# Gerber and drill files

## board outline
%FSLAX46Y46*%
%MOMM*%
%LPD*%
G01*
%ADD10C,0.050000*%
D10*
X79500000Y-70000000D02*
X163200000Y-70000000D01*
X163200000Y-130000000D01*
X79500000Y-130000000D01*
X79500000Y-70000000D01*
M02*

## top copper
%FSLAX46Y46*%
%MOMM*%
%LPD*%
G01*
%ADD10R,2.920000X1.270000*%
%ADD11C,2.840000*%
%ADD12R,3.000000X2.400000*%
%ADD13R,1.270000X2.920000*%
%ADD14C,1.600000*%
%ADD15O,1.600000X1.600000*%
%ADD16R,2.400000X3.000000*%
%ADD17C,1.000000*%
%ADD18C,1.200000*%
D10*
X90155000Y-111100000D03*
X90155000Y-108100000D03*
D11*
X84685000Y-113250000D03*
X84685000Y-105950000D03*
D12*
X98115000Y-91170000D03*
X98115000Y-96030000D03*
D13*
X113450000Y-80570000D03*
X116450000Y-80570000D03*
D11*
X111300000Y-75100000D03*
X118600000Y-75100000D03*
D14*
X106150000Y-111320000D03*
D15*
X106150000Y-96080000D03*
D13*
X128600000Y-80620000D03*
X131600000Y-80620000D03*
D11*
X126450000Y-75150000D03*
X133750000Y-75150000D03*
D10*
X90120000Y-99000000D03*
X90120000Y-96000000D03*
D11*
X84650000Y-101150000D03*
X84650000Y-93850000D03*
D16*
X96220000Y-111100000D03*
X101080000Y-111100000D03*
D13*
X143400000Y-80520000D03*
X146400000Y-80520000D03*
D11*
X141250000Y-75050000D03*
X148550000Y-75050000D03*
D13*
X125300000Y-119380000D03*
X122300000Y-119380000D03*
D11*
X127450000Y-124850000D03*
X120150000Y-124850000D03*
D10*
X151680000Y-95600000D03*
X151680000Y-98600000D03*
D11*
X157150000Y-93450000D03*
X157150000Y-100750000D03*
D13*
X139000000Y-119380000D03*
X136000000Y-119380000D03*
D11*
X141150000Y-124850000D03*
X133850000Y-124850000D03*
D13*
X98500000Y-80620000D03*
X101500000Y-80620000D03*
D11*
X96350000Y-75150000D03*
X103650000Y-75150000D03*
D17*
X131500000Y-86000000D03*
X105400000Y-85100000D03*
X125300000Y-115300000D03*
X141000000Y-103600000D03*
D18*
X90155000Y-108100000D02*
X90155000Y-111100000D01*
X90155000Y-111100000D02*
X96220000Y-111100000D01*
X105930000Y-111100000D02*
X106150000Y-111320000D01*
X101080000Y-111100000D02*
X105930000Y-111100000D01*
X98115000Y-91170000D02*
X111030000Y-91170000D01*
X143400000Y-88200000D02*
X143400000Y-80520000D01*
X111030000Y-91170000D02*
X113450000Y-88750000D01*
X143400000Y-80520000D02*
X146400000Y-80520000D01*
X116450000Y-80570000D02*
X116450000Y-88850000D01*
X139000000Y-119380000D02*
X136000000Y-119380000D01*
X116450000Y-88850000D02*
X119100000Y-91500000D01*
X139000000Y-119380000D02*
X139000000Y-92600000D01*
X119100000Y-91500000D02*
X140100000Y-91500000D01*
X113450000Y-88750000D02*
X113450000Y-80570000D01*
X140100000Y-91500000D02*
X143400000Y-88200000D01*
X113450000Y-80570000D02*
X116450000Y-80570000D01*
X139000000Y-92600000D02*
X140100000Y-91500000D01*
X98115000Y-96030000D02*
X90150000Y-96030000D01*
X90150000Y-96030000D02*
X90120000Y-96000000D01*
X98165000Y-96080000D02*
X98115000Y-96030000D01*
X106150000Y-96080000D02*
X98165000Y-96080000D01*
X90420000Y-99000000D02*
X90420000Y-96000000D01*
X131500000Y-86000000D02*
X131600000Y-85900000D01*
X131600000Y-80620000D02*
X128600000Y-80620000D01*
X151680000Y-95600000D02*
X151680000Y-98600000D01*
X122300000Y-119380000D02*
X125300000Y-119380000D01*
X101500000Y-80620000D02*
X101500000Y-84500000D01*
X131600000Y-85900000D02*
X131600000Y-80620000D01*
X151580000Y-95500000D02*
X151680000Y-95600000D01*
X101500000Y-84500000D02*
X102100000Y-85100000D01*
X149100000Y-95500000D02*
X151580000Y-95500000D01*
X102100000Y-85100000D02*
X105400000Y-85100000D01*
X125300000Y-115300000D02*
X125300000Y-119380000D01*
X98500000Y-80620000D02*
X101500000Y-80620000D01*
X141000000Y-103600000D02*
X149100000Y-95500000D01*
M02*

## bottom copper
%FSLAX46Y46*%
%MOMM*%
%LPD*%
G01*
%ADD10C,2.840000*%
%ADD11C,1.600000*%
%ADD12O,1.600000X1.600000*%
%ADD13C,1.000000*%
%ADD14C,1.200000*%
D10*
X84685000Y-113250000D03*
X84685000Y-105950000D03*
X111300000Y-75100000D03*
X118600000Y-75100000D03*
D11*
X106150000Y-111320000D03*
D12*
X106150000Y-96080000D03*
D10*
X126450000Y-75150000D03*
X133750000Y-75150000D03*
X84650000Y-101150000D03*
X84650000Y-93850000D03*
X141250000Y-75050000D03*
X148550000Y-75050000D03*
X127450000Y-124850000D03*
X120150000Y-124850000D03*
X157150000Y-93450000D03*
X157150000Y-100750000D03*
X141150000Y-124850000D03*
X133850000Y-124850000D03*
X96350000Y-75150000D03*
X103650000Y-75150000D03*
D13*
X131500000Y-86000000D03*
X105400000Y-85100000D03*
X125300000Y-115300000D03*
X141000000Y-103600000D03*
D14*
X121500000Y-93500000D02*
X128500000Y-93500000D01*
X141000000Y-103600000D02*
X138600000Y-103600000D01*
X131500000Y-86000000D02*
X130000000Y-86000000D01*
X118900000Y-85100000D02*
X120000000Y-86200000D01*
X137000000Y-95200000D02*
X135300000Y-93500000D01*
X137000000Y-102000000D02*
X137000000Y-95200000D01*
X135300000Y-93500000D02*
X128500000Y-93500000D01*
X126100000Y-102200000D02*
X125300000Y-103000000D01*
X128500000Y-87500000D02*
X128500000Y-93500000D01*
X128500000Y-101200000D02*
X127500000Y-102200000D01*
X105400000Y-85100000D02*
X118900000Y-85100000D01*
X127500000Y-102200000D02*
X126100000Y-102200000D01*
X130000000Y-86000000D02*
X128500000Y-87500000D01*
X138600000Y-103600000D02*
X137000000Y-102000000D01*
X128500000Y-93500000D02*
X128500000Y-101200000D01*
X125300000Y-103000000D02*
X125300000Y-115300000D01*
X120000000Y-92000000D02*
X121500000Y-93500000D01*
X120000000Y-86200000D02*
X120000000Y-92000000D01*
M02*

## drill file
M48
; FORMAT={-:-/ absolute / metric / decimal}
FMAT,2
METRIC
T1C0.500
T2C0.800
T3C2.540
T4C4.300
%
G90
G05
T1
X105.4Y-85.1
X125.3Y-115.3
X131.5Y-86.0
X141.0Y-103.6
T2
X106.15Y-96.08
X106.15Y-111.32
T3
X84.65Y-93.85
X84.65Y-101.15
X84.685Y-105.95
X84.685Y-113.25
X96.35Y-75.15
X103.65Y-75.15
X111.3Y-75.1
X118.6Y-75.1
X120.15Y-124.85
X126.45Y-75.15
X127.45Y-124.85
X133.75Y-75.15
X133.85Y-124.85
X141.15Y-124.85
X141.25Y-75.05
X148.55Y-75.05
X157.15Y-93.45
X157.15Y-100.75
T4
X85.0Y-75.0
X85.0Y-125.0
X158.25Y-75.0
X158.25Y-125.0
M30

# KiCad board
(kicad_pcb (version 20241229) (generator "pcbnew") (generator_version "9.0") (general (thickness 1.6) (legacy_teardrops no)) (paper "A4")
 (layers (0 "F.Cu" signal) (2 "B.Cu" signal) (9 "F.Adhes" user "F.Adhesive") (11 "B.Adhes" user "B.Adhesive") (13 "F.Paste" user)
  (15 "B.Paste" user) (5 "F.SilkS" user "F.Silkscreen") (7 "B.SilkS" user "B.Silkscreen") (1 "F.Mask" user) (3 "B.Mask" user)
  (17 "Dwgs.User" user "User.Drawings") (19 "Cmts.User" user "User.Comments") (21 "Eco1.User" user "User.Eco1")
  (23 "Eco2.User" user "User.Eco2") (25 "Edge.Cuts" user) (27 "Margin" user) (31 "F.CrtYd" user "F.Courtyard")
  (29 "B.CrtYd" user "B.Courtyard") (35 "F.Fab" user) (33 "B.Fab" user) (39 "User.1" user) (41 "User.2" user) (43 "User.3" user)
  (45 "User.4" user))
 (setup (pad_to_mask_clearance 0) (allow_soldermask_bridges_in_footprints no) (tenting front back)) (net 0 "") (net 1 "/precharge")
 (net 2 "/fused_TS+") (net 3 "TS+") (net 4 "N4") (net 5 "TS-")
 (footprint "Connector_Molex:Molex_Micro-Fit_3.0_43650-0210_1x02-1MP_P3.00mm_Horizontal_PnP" (layer "F.Cu") (at 85.035 109.6 90)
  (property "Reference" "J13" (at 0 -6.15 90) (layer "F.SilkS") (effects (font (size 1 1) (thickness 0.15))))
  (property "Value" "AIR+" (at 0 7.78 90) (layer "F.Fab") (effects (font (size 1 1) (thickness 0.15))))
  (pad "1" smd rect (at -1.5 5.12 90) (size 1.27 2.92) (layers "F.Cu" "F.Mask" "F.Paste") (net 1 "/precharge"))
  (pad "2" smd rect (at 1.5 5.12 90) (size 1.27 2.92) (layers "F.Cu" "F.Mask" "F.Paste") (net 1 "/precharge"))
  (pad "MP" thru_hole circle (at -3.65 -0.35 90) (size 2.84 2.84) (drill 2.54) (layers "*.Cu" "*.Mask") (remove_unused_layers no))
  (pad "MP" thru_hole circle (at 3.65 -0.35 90) (size 2.84 2.84) (drill 2.54) (layers "*.Cu" "*.Mask") (remove_unused_layers no)))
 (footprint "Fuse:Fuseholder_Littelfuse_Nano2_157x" (layer "F.Cu") (at 98.115 93.6 -90)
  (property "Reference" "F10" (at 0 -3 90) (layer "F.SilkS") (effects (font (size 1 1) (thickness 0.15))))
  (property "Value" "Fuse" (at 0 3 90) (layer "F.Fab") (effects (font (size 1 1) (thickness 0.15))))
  (pad "1" smd rect (at -2.43 0 270) (size 2.4 3) (layers "F.Cu" "F.Mask" "F.Paste") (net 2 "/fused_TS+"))
  (pad "2" smd rect (at 2.43 0 270) (size 2.4 3) (layers "F.Cu" "F.Mask" "F.Paste") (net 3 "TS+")))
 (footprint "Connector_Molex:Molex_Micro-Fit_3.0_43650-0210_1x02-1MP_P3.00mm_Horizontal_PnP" (layer "F.Cu") (at 114.95 75.45)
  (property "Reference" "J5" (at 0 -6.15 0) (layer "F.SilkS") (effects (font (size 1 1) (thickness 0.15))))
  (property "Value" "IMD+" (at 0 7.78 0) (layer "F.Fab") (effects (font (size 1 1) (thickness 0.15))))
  (pad "1" smd rect (at -1.5 5.12) (size 1.27 2.92) (layers "F.Cu" "F.Mask" "F.Paste") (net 2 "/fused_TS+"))
  (pad "2" smd rect (at 1.5 5.12) (size 1.27 2.92) (layers "F.Cu" "F.Mask" "F.Paste") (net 2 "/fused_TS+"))
  (pad "MP" thru_hole circle (at -3.65 -0.35) (size 2.84 2.84) (drill 2.54) (layers "*.Cu" "*.Mask") (remove_unused_layers no))
  (pad "MP" thru_hole circle (at 3.65 -0.35) (size 2.84 2.84) (drill 2.54) (layers "*.Cu" "*.Mask") (remove_unused_layers no)))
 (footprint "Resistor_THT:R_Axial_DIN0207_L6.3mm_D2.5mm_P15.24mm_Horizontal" (layer "F.Cu") (at 106.15 111.32 90)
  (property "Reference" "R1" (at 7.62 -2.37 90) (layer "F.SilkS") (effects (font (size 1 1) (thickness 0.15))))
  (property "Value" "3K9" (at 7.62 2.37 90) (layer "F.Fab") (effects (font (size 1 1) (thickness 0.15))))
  (pad "1" thru_hole circle (at 0 0 90) (size 1.6 1.6) (drill 0.8) (layers "*.Cu" "*.Mask") (remove_unused_layers no) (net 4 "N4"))
  (pad "2" thru_hole oval (at 15.24 0 90) (size 1.6 1.6) (drill 0.8) (layers "*.Cu" "*.Mask") (remove_unused_layers no) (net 3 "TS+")))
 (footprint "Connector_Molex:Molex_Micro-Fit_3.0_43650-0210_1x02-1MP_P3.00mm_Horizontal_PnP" (layer "F.Cu") (at 130.1 75.5)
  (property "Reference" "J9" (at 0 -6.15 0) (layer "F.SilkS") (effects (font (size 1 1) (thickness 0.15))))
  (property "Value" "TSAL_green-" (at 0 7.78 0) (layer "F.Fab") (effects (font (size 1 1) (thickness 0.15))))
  (pad "1" smd rect (at -1.5 5.12) (size 1.27 2.92) (layers "F.Cu" "F.Mask" "F.Paste") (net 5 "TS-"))
  (pad "2" smd rect (at 1.5 5.12) (size 1.27 2.92) (layers "F.Cu" "F.Mask" "F.Paste") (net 5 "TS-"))
  (pad "MP" thru_hole circle (at -3.65 -0.35) (size 2.84 2.84) (drill 2.54) (layers "*.Cu" "*.Mask") (remove_unused_layers no))
  (pad "MP" thru_hole circle (at 3.65 -0.35) (size 2.84 2.84) (drill 2.54) (layers "*.Cu" "*.Mask") (remove_unused_layers no)))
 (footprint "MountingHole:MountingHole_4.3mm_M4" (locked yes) (layer "F.Cu") (at 85 75)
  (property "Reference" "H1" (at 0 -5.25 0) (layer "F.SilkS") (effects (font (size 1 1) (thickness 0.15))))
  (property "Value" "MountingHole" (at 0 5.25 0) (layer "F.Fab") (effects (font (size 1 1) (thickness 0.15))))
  (pad "" np_thru_hole circle (at 0 0) (size 4.3 4.3) (drill 4.3) (layers "*.Cu" "*.Mask")))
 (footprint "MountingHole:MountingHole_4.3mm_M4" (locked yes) (layer "F.Cu") (at 85 125)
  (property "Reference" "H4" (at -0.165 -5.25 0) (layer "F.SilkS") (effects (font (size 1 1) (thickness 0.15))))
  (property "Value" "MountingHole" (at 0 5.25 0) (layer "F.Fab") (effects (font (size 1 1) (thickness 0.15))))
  (pad "" np_thru_hole circle (at 0 0) (size 4.3 4.3) (drill 4.3) (layers "*.Cu" "*.Mask")))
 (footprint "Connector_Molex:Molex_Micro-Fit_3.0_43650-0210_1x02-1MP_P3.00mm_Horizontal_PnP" (layer "F.Cu") (at 85 97.5 90)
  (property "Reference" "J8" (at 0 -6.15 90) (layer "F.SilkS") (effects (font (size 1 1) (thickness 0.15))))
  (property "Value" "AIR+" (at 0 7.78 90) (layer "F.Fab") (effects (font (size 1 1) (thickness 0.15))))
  (pad "1" smd rect (at -1.5 5.12 90) (size 1.27 2.92) (layers "F.Cu" "F.Mask" "F.Paste") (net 3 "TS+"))
  (pad "2" smd rect (at 1.5 5.12 90) (size 1.27 2.92) (layers "F.Cu" "F.Mask" "F.Paste") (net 3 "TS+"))
  (pad "MP" thru_hole circle (at -3.65 -0.35 90) (size 2.84 2.84) (drill 2.54) (layers "*.Cu" "*.Mask") (remove_unused_layers no))
  (pad "MP" thru_hole circle (at 3.65 -0.35 90) (size 2.84 2.84) (drill 2.54) (layers "*.Cu" "*.Mask") (remove_unused_layers no)))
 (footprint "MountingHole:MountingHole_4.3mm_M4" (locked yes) (layer "F.Cu") (at 158.25 75)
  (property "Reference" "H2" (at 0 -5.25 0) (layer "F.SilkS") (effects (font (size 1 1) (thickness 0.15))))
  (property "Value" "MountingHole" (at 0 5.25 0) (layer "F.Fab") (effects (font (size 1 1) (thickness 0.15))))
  (pad "" np_thru_hole circle (at 0 0) (size 4.3 4.3) (drill 4.3) (layers "*.Cu" "*.Mask")))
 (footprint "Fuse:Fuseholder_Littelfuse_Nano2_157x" (layer "F.Cu") (at 98.65 111.1)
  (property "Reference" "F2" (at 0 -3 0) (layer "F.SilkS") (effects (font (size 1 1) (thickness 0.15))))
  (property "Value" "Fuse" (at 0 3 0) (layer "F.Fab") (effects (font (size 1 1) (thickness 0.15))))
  (pad "1" smd rect (at -2.43 0) (size 2.4 3) (layers "F.Cu" "F.Mask" "F.Paste") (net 1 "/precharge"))
  (pad "2" smd rect (at 2.43 0) (size 2.4 3) (layers "F.Cu" "F.Mask" "F.Paste") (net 4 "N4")))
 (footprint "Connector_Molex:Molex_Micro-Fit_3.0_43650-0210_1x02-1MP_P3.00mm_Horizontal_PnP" (layer "F.Cu") (at 144.9 75.4)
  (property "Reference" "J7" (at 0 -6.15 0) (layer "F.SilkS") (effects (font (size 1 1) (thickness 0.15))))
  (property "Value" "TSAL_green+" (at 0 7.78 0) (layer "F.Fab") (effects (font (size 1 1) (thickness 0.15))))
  (pad "1" smd rect (at -1.5 5.12) (size 1.27 2.92) (layers "F.Cu" "F.Mask" "F.Paste") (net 2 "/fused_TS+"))
  (pad "2" smd rect (at 1.5 5.12) (size 1.27 2.92) (layers "F.Cu" "F.Mask" "F.Paste") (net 2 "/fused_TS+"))
  (pad "MP" thru_hole circle (at -3.65 -0.35) (size 2.84 2.84) (drill 2.54) (layers "*.Cu" "*.Mask") (remove_unused_layers no))
  (pad "MP" thru_hole circle (at 3.65 -0.35) (size 2.84 2.84) (drill 2.54) (layers "*.Cu" "*.Mask") (remove_unused_layers no)))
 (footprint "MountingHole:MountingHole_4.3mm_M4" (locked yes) (layer "F.Cu") (at 158.25 125)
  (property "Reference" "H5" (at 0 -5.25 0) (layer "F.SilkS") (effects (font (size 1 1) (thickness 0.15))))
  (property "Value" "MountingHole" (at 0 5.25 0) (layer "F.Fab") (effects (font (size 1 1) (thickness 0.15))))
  (pad "" np_thru_hole circle (at 0 0) (size 4.3 4.3) (drill 4.3) (layers "*.Cu" "*.Mask")))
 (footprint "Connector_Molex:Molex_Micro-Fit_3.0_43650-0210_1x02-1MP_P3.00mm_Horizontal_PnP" (layer "F.Cu") (at 123.8 124.5 180)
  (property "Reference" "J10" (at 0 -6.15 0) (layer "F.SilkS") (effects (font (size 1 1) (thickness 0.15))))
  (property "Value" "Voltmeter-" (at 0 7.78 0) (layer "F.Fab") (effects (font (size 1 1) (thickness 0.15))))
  (pad "1" smd rect (at -1.5 5.12 180) (size 1.27 2.92) (layers "F.Cu" "F.Mask" "F.Paste") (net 5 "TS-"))
  (pad "2" smd rect (at 1.5 5.12 180) (size 1.27 2.92) (layers "F.Cu" "F.Mask" "F.Paste") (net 5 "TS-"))
  (pad "MP" thru_hole circle (at -3.65 -0.35 180) (size 2.84 2.84) (drill 2.54) (layers "*.Cu" "*.Mask") (remove_unused_layers no))
  (pad "MP" thru_hole circle (at 3.65 -0.35 180) (size 2.84 2.84) (drill 2.54) (layers "*.Cu" "*.Mask") (remove_unused_layers no)))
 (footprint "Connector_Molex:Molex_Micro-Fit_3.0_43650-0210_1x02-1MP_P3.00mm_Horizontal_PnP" (layer "F.Cu") (at 156.8 97.1 -90)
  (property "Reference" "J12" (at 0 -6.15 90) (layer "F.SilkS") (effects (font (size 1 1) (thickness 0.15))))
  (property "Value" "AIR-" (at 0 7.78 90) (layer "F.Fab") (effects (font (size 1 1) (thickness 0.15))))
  (pad "1" smd rect (at -1.5 5.12 270) (size 1.27 2.92) (layers "F.Cu" "F.Mask" "F.Paste") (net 5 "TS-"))
  (pad "2" smd rect (at 1.5 5.12 270) (size 1.27 2.92) (layers "F.Cu" "F.Mask" "F.Paste") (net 5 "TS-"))
  (pad "MP" thru_hole circle (at -3.65 -0.35 270) (size 2.84 2.84) (drill 2.54) (layers "*.Cu" "*.Mask") (remove_unused_layers no))
  (pad "MP" thru_hole circle (at 3.65 -0.35 270) (size 2.84 2.84) (drill 2.54) (layers "*.Cu" "*.Mask") (remove_unused_layers no)))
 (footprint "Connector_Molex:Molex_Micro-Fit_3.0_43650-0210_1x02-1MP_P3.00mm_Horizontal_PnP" (layer "F.Cu") (at 137.5 124.5 180)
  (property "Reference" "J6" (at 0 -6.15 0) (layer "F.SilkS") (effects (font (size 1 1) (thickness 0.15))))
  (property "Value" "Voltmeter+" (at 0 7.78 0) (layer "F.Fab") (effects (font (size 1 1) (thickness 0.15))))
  (pad "1" smd rect (at -1.5 5.12 180) (size 1.27 2.92) (layers "F.Cu" "F.Mask" "F.Paste") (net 2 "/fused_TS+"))
  (pad "2" smd rect (at 1.5 5.12 180) (size 1.27 2.92) (layers "F.Cu" "F.Mask" "F.Paste") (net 2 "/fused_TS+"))
  (pad "MP" thru_hole circle (at -3.65 -0.35 180) (size 2.84 2.84) (drill 2.54) (layers "*.Cu" "*.Mask") (remove_unused_layers no))
  (pad "MP" thru_hole circle (at 3.65 -0.35 180) (size 2.84 2.84) (drill 2.54) (layers "*.Cu" "*.Mask") (remove_unused_layers no)))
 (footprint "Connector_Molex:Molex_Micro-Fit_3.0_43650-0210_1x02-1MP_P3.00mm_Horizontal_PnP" (layer "F.Cu") (at 100 75.5)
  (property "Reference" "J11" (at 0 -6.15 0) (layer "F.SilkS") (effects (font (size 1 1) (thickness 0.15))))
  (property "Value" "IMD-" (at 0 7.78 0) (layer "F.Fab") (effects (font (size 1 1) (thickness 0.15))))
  (pad "1" smd rect (at -1.5 5.12) (size 1.27 2.92) (layers "F.Cu" "F.Mask" "F.Paste") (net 5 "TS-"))
  (pad "2" smd rect (at 1.5 5.12) (size 1.27 2.92) (layers "F.Cu" "F.Mask" "F.Paste") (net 5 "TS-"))
  (pad "MP" thru_hole circle (at -3.65 -0.35) (size 2.84 2.84) (drill 2.54) (layers "*.Cu" "*.Mask") (remove_unused_layers no))
  (pad "MP" thru_hole circle (at 3.65 -0.35) (size 2.84 2.84) (drill 2.54) (layers "*.Cu" "*.Mask") (remove_unused_layers no)))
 (gr_rect (start 79.5 70) (end 163.2 130) (stroke (width 0.05) (type default)) (fill no) (layer "Edge.Cuts"))
 (segment (start 90.155 108.1) (end 90.155 111.1) (width 1.2) (layer "F.Cu") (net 1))
 (segment (start 90.155 111.1) (end 96.22 111.1) (width 1.2) (layer "F.Cu") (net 1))
 (segment (start 105.93 111.1) (end 106.15 111.32) (width 1.2) (layer "F.Cu") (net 4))
 (segment (start 101.08 111.1) (end 105.93 111.1) (width 1.2) (layer "F.Cu") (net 4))
 (segment (start 98.115 91.17) (end 111.03 91.17) (width 1.2) (layer "F.Cu") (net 2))
 (segment (start 143.4 88.2) (end 143.4 80.52) (width 1.2) (layer "F.Cu") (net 2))
 (segment (start 111.03 91.17) (end 113.45 88.75) (width 1.2) (layer "F.Cu") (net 2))
 (segment (start 143.4 80.52) (end 146.4 80.52) (width 1.2) (layer "F.Cu") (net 2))
 (segment (start 116.45 80.57) (end 116.45 88.85) (width 1.2) (layer "F.Cu") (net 2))
 (segment (start 139 119.38) (end 136 119.38) (width 1.2) (layer "F.Cu") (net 2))
 (segment (start 116.45 88.85) (end 119.1 91.5) (width 1.2) (layer "F.Cu") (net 2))
 (segment (start 139 119.38) (end 139 92.6) (width 1.2) (layer "F.Cu") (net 2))
 (segment (start 119.1 91.5) (end 140.1 91.5) (width 1.2) (layer "F.Cu") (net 2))
 (segment (start 113.45 88.75) (end 113.45 80.57) (width 1.2) (layer "F.Cu") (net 2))
 (segment (start 140.1 91.5) (end 143.4 88.2) (width 1.2) (layer "F.Cu") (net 2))
 (segment (start 113.45 80.57) (end 116.45 80.57) (width 1.2) (layer "F.Cu") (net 2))
 (segment (start 139 92.6) (end 140.1 91.5) (width 1.2) (layer "F.Cu") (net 2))
 (segment (start 98.115 96.03) (end 90.15 96.03) (width 1.2) (layer "F.Cu") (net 3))
 (segment (start 90.15 96.03) (end 90.12 96) (width 1.2) (layer "F.Cu") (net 3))
 (segment (start 98.165 96.08) (end 98.115 96.03) (width 1.2) (layer "F.Cu") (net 3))
 (segment (start 106.15 96.08) (end 98.165 96.08) (width 1.2) (layer "F.Cu") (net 3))
 (segment (start 90.42 99) (end 90.42 96) (width 1.2) (layer "F.Cu") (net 3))
 (segment (start 131.5 86) (end 131.6 85.9) (width 1.2) (layer "F.Cu") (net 5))
 (segment (start 131.6 80.62) (end 128.6 80.62) (width 1.2) (layer "F.Cu") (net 5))
 (segment (start 151.68 95.6) (end 151.68 98.6) (width 1.2) (layer "F.Cu") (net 5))
 (segment (start 122.3 119.38) (end 125.3 119.38) (width 1.2) (layer "F.Cu") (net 5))
 (segment (start 101.5 80.62) (end 101.5 84.5) (width 1.2) (layer "F.Cu") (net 5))
 (segment (start 131.6 85.9) (end 131.6 80.62) (width 1.2) (layer "F.Cu") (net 5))
 (segment (start 151.58 95.5) (end 151.68 95.6) (width 1.2) (layer "F.Cu") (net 5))
 (segment (start 101.5 84.5) (end 102.1 85.1) (width 1.2) (layer "F.Cu") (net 5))
 (segment (start 149.1 95.5) (end 151.58 95.5) (width 1.2) (layer "F.Cu") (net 5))
 (segment (start 102.1 85.1) (end 105.4 85.1) (width 1.2) (layer "F.Cu") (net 5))
 (segment (start 125.3 115.3) (end 125.3 119.38) (width 1.2) (layer "F.Cu") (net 5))
 (segment (start 98.5 80.62) (end 101.5 80.62) (width 1.2) (layer "F.Cu") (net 5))
 (segment (start 141 103.6) (end 149.1 95.5) (width 1.2) (layer "F.Cu") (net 5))
 (via (at 131.5 86) (size 1) (drill 0.5) (layers "F.Cu" "B.Cu") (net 5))
 (via (at 105.4 85.1) (size 1) (drill 0.5) (layers "F.Cu" "B.Cu") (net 5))
 (via (at 125.3 115.3) (size 1) (drill 0.5) (layers "F.Cu" "B.Cu") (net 5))
 (via (at 141 103.6) (size 1) (drill 0.5) (layers "F.Cu" "B.Cu") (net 5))
 (segment (start 121.5 93.5) (end 128.5 93.5) (width 1.2) (layer "B.Cu") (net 5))
 (segment (start 141 103.6) (end 138.6 103.6) (width 1.2) (layer "B.Cu") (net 5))
 (segment (start 131.5 86) (end 130 86) (width 1.2) (layer "B.Cu") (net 5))
 (segment (start 118.9 85.1) (end 120 86.2) (width 1.2) (layer "B.Cu") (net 5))
 (segment (start 137 95.2) (end 135.3 93.5) (width 1.2) (layer "B.Cu") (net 5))
 (segment (start 137 102) (end 137 95.2) (width 1.2) (layer "B.Cu") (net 5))
 (segment (start 135.3 93.5) (end 128.5 93.5) (width 1.2) (layer "B.Cu") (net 5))
 (segment (start 126.1 102.2) (end 125.3 103) (width 1.2) (layer "B.Cu") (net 5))
 (segment (start 128.5 87.5) (end 128.5 93.5) (width 1.2) (layer "B.Cu") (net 5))
 (segment (start 128.5 101.2) (end 127.5 102.2) (width 1.2) (layer "B.Cu") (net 5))
 (segment (start 105.4 85.1) (end 118.9 85.1) (width 1.2) (layer "B.Cu") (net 5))
 (segment (start 127.5 102.2) (end 126.1 102.2) (width 1.2) (layer "B.Cu") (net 5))
 (segment (start 130 86) (end 128.5 87.5) (width 1.2) (layer "B.Cu") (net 5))
 (segment (start 138.6 103.6) (end 137 102) (width 1.2) (layer "B.Cu") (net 5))
 (segment (start 128.5 93.5) (end 128.5 101.2) (width 1.2) (layer "B.Cu") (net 5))
 (segment (start 125.3 103) (end 125.3 115.3) (width 1.2) (layer "B.Cu") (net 5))
 (segment (start 120 92) (end 121.5 93.5) (width 1.2) (layer "B.Cu") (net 5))
 (segment (start 120 86.2) (end 120 92) (width 1.2) (layer "B.Cu") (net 5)))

